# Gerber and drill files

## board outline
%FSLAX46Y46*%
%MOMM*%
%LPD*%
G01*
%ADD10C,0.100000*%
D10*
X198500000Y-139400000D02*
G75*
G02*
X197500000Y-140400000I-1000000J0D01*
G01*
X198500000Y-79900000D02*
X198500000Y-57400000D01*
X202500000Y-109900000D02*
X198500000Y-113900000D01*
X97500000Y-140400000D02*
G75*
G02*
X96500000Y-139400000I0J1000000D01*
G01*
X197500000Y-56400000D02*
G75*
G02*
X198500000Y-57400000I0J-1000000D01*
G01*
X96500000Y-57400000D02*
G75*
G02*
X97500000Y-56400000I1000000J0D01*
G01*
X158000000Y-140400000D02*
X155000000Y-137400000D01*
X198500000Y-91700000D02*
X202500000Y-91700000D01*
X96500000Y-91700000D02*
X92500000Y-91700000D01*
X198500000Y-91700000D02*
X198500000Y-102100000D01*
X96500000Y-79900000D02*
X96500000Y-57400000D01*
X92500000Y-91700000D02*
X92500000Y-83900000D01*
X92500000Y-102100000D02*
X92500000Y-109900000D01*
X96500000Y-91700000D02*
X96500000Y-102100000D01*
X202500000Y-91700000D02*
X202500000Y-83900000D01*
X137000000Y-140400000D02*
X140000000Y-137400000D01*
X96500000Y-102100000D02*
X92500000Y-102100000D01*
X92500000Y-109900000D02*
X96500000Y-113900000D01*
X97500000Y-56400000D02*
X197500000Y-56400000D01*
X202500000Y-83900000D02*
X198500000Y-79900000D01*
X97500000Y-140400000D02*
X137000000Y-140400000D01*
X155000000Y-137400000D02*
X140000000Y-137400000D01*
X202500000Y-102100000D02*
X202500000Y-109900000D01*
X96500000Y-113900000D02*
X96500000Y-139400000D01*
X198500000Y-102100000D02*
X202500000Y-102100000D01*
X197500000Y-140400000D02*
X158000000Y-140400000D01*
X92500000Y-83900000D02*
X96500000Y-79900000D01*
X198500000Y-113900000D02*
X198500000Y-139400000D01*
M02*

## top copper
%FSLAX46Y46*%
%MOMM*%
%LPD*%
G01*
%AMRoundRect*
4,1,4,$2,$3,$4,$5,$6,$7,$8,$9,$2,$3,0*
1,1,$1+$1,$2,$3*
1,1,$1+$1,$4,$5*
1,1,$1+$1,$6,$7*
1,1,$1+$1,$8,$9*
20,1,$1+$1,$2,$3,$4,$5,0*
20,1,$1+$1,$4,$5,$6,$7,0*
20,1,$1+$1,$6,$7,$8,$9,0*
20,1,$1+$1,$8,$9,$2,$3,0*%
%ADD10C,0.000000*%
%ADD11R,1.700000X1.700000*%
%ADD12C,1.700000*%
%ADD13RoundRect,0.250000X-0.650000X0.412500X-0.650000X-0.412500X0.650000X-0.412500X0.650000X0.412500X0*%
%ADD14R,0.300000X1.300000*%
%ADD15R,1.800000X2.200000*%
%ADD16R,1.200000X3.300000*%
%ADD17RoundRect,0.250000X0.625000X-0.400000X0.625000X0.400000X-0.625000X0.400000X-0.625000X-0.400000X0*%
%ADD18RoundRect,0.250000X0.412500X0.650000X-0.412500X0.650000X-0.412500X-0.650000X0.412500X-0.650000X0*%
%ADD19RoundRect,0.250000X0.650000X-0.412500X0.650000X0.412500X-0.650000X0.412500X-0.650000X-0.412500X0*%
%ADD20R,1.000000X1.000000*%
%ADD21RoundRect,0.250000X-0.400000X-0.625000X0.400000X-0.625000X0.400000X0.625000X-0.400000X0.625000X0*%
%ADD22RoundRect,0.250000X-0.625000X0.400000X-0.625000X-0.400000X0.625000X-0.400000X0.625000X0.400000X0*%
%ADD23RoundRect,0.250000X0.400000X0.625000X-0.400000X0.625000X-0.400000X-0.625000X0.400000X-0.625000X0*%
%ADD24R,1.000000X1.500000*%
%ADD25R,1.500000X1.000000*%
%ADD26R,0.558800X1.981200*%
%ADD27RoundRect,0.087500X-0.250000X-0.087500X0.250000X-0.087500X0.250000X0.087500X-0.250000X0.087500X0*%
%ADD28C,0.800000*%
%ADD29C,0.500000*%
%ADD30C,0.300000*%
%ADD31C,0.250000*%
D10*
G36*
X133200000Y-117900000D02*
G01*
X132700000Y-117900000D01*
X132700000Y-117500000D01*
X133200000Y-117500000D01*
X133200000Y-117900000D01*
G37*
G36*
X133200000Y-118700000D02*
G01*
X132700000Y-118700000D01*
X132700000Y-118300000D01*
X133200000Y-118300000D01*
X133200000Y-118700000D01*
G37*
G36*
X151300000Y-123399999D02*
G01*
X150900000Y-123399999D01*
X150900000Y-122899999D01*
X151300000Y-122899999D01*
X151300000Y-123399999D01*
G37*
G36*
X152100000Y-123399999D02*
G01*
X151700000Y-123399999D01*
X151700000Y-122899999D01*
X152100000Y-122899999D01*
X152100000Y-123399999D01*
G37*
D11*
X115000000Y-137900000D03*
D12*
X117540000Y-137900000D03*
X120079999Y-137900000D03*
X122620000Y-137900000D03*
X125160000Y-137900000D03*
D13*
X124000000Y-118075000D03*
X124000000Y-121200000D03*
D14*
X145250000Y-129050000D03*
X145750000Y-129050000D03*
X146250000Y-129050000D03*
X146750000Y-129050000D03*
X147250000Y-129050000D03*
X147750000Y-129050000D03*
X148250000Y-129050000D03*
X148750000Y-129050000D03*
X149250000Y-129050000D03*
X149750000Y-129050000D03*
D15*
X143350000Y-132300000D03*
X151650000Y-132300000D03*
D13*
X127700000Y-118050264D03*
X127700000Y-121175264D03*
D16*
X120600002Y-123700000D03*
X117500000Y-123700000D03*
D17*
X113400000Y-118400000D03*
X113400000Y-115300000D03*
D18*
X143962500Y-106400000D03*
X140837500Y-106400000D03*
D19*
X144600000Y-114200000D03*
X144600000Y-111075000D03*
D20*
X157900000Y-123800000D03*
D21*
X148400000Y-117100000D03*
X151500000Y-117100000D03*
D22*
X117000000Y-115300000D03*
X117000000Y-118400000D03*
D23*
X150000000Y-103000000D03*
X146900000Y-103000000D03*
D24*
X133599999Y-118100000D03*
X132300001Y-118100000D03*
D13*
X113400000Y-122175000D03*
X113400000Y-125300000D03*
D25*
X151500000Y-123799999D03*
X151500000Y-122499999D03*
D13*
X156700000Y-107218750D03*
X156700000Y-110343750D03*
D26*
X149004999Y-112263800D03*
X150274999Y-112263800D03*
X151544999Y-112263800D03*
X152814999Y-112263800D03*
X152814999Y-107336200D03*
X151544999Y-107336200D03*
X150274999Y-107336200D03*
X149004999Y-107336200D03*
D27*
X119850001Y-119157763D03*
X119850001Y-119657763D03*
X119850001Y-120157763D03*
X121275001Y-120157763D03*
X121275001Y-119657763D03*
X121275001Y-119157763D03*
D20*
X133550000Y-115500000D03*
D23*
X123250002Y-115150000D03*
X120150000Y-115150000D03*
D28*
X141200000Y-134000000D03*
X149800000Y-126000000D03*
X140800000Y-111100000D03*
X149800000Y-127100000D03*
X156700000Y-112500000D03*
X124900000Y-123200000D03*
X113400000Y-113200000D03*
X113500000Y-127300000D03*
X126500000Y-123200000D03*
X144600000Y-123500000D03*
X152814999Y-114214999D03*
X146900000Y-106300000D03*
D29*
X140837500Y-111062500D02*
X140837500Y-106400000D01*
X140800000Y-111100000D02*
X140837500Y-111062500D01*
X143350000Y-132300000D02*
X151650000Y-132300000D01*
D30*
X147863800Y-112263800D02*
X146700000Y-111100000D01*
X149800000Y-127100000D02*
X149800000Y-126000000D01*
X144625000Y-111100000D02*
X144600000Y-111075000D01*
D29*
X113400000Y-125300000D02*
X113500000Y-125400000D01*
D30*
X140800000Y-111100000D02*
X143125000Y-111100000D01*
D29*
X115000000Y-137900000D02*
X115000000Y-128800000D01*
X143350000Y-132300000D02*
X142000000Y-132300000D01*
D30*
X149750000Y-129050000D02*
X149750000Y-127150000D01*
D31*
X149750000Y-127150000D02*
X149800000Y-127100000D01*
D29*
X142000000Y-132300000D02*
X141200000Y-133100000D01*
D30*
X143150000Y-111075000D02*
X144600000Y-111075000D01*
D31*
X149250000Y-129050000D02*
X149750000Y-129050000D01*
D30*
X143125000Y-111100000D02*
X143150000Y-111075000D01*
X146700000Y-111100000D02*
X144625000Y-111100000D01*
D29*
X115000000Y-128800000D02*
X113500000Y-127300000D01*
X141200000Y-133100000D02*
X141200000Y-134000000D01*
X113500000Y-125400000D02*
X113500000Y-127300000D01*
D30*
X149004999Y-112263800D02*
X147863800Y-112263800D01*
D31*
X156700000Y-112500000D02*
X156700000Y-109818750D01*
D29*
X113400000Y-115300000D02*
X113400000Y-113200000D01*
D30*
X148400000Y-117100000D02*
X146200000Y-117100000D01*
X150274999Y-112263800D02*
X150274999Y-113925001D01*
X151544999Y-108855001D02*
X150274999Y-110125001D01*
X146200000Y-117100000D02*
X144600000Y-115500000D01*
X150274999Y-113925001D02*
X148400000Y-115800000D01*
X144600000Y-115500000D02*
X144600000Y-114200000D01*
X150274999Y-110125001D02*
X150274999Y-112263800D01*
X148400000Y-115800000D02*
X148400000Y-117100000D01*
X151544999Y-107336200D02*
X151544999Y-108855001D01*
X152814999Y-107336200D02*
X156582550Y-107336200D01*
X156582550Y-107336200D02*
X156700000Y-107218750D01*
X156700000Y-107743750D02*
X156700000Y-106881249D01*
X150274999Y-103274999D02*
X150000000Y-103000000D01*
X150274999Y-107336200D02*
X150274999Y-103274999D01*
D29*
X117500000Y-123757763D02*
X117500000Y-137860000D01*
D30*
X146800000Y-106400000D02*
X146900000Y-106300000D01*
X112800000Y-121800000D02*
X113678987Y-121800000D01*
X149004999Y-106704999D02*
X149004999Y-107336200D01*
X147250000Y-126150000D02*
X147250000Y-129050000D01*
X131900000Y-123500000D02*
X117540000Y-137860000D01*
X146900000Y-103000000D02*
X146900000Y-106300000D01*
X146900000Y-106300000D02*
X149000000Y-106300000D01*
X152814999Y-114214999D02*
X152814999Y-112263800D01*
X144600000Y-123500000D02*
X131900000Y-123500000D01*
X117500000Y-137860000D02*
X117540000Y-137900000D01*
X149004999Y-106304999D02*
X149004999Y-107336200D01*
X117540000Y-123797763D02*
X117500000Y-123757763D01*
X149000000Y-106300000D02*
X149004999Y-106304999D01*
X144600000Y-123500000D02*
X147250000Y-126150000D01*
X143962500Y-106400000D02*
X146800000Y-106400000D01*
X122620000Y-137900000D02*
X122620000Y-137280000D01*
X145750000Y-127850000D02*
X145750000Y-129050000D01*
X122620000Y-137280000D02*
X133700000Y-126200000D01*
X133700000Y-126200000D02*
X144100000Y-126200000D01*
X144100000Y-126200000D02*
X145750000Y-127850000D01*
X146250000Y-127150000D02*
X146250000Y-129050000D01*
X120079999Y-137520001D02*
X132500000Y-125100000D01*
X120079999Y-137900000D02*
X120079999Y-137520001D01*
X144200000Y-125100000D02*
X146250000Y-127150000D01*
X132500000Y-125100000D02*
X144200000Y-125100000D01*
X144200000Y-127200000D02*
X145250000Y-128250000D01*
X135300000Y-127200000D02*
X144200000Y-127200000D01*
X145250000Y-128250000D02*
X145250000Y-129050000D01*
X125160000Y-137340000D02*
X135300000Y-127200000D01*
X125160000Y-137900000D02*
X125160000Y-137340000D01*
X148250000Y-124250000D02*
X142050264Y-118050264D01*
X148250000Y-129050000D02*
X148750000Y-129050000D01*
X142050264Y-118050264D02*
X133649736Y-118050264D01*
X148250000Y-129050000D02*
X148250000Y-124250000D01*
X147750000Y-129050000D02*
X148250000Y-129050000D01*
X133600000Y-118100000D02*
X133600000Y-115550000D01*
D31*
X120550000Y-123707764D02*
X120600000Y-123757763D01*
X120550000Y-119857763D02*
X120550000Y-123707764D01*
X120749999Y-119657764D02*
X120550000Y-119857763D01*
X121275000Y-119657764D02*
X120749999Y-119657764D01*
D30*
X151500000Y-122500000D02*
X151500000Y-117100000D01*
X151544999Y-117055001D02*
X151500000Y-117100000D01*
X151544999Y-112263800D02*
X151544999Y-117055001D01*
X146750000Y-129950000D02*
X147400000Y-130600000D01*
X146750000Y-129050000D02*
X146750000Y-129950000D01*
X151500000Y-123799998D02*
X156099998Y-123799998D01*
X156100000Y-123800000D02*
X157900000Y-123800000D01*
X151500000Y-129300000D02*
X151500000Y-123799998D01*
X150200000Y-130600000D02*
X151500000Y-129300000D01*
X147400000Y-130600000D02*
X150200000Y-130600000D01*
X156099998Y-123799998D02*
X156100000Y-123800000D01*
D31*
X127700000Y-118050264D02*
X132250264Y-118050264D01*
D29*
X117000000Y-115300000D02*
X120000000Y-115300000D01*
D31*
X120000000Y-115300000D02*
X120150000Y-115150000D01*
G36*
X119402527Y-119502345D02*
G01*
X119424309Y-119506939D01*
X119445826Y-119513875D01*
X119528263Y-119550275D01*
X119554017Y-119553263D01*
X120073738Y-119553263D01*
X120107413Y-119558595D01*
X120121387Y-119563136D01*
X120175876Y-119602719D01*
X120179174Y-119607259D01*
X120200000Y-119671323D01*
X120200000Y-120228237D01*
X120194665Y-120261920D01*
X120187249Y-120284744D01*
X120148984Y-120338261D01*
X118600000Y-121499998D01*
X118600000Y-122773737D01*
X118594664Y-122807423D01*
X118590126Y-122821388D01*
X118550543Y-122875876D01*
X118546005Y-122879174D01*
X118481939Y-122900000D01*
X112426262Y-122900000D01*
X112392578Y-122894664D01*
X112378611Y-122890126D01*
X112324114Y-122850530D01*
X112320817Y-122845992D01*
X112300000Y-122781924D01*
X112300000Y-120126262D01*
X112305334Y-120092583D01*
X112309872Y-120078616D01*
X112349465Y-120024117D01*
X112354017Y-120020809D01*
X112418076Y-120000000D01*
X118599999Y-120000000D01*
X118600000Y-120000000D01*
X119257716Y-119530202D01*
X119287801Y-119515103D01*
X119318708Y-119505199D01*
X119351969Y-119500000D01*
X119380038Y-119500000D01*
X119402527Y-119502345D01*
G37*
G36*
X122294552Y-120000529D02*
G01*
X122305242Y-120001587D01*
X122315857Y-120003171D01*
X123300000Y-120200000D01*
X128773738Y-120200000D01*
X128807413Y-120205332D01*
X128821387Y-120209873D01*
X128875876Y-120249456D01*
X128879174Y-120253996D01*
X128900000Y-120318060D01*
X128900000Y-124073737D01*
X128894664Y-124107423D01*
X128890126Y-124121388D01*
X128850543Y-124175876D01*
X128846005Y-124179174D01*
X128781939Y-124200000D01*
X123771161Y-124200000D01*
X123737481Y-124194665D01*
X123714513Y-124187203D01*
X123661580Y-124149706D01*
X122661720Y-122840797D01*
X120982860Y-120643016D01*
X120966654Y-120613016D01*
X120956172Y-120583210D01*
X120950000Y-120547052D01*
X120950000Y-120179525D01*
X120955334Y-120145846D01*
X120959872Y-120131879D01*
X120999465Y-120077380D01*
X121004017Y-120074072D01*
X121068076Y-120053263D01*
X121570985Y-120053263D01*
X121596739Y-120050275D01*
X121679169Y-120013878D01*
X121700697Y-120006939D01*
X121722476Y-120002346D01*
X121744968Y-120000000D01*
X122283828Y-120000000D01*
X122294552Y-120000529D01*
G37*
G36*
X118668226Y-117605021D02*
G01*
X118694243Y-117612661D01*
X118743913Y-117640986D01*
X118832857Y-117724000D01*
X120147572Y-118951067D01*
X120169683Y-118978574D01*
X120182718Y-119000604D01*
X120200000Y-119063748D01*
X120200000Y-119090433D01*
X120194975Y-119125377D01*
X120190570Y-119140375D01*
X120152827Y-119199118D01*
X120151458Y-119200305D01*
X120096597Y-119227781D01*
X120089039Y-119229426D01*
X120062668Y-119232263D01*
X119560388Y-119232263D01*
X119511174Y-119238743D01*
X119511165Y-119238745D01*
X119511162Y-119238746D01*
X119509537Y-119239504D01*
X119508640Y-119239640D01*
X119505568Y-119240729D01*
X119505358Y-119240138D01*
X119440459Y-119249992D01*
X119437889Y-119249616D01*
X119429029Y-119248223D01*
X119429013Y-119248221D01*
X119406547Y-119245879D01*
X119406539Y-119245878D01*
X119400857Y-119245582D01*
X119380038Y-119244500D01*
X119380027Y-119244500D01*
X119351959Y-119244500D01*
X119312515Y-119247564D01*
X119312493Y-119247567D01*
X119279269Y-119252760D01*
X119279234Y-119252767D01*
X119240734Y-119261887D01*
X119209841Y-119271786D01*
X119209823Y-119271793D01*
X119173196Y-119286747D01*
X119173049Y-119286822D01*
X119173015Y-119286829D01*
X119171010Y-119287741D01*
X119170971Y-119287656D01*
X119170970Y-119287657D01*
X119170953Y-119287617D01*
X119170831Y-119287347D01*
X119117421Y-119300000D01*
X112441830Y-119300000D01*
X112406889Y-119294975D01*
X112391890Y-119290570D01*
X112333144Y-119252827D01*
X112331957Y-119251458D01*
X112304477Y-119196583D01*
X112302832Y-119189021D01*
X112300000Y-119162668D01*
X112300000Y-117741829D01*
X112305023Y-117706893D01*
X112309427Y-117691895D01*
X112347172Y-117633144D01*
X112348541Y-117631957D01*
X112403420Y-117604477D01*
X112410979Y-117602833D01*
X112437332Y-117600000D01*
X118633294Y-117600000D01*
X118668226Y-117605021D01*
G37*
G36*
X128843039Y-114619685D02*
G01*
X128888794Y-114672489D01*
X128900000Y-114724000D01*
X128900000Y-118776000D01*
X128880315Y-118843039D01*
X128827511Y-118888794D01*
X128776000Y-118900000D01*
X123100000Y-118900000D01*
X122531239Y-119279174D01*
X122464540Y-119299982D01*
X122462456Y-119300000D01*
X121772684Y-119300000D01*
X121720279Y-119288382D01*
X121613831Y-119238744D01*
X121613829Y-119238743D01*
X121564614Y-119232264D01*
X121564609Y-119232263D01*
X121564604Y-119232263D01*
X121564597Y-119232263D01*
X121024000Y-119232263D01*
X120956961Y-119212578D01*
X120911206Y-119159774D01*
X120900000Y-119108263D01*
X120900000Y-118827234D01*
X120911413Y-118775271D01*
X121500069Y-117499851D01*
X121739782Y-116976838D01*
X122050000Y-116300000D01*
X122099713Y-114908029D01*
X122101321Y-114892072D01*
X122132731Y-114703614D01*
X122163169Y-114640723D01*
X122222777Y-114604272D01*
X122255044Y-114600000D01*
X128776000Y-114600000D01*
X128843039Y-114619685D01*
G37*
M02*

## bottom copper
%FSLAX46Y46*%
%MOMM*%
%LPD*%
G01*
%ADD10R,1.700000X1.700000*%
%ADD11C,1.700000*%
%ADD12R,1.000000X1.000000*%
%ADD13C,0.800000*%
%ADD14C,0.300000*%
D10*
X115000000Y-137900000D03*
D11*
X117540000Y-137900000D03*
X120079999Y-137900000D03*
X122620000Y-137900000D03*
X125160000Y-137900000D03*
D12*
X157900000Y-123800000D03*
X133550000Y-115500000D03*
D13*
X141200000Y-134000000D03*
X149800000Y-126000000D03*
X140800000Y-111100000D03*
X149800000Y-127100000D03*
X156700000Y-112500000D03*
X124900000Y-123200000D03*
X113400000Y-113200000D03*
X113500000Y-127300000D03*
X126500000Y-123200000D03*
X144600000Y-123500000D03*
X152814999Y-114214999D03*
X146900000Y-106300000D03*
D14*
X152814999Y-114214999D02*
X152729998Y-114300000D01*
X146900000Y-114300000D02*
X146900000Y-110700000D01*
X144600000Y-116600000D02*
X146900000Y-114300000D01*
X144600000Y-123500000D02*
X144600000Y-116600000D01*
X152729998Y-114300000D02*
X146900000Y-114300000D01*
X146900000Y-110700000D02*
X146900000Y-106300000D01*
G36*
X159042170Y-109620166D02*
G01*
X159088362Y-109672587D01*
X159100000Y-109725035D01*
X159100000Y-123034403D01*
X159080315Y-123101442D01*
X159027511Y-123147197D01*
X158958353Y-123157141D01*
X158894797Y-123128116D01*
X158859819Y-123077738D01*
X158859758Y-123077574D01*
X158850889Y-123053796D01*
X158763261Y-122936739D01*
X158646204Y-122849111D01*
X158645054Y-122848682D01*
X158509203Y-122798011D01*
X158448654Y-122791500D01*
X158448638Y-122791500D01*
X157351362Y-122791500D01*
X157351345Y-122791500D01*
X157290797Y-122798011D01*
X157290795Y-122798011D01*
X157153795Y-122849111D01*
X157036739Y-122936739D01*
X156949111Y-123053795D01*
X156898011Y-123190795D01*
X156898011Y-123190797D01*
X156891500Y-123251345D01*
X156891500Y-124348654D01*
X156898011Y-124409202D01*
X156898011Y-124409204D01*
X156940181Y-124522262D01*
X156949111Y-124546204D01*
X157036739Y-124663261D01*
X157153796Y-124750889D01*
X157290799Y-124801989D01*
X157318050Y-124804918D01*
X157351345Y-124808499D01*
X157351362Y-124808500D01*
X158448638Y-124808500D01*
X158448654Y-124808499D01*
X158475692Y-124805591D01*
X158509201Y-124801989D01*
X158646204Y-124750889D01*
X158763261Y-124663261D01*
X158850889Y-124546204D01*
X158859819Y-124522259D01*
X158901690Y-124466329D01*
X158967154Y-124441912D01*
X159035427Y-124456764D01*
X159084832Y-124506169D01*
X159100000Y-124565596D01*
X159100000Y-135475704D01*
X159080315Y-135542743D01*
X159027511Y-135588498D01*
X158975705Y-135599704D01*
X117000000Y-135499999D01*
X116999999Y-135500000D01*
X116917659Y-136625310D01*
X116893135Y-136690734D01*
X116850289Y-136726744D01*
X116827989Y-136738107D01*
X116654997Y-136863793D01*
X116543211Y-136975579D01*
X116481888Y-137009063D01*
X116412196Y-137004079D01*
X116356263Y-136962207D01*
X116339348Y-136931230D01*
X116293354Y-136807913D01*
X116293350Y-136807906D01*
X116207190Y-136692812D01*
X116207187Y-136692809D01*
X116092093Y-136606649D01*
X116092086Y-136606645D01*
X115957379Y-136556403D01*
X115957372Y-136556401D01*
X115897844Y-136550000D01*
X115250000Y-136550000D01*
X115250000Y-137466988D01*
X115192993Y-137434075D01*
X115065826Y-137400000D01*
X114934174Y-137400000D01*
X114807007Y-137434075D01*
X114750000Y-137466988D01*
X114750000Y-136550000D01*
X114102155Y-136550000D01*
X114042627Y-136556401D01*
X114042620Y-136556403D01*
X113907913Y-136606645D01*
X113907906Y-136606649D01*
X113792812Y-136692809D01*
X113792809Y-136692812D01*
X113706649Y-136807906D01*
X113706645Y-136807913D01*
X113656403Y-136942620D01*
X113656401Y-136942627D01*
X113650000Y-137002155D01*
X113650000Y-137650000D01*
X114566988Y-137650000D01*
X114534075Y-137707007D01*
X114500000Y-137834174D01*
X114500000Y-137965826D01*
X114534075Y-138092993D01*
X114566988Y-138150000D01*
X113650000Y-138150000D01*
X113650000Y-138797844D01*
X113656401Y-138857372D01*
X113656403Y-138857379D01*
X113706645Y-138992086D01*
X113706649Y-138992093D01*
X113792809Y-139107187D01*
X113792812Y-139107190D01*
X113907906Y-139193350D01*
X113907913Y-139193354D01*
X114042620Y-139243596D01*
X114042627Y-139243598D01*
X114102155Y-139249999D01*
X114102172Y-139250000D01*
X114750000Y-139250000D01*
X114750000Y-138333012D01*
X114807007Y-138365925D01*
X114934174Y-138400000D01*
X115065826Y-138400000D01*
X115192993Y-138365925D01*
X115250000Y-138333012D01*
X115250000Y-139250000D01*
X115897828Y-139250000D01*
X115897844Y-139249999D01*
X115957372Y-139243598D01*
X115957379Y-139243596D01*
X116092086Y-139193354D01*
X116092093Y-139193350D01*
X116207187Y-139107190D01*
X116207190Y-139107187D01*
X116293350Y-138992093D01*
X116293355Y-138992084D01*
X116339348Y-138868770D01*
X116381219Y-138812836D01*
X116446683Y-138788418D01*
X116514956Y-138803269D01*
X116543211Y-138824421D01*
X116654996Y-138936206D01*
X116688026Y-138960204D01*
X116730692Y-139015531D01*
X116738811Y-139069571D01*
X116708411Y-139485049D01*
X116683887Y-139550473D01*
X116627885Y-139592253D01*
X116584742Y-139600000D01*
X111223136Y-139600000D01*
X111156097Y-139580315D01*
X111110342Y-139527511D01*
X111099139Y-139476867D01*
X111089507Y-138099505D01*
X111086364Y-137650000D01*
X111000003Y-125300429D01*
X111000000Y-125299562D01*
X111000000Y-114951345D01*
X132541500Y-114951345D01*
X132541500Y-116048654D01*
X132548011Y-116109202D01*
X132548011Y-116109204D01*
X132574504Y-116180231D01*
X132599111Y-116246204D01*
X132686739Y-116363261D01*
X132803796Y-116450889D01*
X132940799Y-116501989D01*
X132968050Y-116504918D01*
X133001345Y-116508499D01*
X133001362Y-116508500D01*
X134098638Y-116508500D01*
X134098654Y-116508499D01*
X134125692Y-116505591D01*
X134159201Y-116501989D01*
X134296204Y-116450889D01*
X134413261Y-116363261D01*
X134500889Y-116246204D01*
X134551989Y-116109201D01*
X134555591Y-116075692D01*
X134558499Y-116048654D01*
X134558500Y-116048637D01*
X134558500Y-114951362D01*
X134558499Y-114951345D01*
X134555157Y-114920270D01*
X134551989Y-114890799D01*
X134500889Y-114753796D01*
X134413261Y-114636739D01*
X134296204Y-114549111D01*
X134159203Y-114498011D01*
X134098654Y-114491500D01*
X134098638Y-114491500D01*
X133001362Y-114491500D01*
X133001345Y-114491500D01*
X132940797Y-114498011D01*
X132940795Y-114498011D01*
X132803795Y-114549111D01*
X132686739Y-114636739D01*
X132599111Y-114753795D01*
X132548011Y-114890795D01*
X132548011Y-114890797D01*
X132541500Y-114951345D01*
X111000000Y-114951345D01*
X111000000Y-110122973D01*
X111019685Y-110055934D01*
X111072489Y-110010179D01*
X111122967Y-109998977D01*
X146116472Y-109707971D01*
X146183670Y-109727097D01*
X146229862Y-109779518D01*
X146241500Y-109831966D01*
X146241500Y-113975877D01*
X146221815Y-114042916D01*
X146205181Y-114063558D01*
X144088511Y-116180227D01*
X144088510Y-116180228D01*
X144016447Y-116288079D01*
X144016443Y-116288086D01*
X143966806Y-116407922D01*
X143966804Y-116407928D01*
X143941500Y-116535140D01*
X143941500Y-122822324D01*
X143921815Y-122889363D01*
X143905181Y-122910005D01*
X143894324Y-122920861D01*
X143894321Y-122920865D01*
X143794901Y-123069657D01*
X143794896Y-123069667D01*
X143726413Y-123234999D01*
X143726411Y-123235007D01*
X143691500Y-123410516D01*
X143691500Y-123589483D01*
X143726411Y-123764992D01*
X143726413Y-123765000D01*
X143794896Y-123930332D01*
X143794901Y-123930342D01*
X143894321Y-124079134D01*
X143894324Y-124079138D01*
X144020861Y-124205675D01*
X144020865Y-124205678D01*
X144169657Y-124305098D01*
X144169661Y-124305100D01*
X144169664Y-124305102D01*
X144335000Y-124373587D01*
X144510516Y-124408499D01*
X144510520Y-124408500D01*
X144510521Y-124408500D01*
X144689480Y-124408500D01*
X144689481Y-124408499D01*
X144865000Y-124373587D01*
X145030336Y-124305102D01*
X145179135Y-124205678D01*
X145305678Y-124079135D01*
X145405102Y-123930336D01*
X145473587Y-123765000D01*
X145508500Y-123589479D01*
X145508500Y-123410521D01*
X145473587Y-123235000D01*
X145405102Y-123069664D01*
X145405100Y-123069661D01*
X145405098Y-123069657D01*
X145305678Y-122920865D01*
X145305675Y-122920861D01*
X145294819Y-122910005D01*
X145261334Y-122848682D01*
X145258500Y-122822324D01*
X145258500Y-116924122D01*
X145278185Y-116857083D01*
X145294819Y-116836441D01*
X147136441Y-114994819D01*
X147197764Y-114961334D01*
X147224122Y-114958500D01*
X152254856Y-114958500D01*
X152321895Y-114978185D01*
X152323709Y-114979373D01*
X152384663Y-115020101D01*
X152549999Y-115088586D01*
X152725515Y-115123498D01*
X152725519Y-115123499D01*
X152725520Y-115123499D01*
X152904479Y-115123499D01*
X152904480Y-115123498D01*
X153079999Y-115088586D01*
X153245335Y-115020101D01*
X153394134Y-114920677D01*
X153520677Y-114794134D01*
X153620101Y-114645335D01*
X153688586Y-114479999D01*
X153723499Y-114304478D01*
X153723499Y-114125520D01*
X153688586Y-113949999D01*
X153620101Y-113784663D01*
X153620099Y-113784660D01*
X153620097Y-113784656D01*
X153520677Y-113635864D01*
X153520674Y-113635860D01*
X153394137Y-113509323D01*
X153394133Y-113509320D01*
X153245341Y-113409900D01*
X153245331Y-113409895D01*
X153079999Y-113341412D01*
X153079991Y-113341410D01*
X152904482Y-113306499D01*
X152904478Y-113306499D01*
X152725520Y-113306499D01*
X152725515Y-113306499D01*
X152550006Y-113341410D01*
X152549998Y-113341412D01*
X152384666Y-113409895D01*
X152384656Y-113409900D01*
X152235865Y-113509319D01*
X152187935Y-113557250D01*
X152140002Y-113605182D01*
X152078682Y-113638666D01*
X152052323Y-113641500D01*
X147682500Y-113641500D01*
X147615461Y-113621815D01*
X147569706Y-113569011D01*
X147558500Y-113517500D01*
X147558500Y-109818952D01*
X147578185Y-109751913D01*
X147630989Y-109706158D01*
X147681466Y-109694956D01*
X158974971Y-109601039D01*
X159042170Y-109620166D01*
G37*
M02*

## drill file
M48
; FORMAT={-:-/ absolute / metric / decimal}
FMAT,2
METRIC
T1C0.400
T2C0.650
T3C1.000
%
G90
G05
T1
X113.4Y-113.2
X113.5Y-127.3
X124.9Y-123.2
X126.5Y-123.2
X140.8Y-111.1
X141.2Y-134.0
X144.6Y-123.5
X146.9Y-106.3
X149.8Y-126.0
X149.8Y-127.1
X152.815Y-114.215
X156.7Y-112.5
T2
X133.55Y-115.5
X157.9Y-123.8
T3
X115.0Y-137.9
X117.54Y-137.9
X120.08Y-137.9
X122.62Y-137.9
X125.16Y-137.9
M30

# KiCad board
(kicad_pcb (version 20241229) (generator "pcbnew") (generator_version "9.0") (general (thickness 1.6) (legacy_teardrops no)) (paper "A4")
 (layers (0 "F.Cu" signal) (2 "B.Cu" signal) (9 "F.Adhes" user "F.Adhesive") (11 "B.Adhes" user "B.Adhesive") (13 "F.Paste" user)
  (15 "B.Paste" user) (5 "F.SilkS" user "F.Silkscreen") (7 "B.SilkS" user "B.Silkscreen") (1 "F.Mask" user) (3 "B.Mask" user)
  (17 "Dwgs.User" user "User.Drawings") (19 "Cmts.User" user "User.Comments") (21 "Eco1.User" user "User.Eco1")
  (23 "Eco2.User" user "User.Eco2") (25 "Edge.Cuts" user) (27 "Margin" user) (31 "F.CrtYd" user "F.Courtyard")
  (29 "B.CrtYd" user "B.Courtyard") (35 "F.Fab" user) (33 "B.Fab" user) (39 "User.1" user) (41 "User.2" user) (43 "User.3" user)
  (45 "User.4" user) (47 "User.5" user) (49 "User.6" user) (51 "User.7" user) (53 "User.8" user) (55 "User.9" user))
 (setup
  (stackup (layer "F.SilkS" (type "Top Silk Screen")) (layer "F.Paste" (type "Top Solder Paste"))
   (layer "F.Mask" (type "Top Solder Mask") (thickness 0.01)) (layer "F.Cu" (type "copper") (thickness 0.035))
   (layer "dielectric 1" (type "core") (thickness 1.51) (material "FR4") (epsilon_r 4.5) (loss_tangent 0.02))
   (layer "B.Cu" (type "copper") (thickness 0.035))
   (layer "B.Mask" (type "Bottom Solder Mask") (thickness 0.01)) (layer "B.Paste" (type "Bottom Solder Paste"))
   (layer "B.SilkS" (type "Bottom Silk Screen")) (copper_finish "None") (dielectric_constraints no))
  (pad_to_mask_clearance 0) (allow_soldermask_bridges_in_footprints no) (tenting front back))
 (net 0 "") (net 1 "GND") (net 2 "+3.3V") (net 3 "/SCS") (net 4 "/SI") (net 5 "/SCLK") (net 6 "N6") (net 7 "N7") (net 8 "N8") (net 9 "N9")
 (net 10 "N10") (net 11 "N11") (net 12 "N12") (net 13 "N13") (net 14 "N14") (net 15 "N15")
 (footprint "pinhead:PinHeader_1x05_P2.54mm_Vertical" (layer "F.Cu") (at 115 137.9 90)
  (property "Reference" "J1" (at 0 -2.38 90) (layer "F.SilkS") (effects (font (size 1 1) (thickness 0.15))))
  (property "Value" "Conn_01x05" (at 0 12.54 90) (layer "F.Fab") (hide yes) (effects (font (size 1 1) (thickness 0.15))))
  (pad "1" thru_hole rect (at 0 0 90) (size 1.7 1.7) (drill 1) (layers "*.Cu" "*.Mask") (remove_unused_layers no) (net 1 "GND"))
  (pad "2" thru_hole circle (at 0 2.54 90) (size 1.7 1.7) (drill 1) (layers "*.Cu" "*.Mask") (remove_unused_layers no) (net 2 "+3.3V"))
  (pad "3" thru_hole circle (at 0 5.079999 90) (size 1.7 1.7) (drill 1) (layers "*.Cu" "*.Mask") (remove_unused_layers no) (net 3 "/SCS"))
  (pad "4" thru_hole circle (at 0 7.62 90) (size 1.7 1.7) (drill 1) (layers "*.Cu" "*.Mask") (remove_unused_layers no) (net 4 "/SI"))
  (pad "5" thru_hole circle (at 0 10.16 90) (size 1.7 1.7) (drill 1) (layers "*.Cu" "*.Mask") (remove_unused_layers no) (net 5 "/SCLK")))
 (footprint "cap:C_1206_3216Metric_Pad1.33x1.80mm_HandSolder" (layer "F.Cu") (at 124 119.6375 -90)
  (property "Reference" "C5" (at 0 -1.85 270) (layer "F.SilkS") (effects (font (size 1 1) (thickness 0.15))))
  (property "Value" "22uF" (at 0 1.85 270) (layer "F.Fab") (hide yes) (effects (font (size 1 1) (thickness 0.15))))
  (pad "1" smd roundrect (at -1.5625 0 270) (size 1.325 1.8) (layers "F.Cu" "F.Mask" "F.Paste") (roundrect_rratio 0.188679) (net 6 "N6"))
  (pad "2" smd roundrect (at 1.5625 0 270) (size 1.325 1.8) (layers "F.Cu" "F.Mask" "F.Paste") (roundrect_rratio 0.188679) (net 1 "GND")))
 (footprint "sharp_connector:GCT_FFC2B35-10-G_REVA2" (layer "F.Cu") (at 147.5 132.3)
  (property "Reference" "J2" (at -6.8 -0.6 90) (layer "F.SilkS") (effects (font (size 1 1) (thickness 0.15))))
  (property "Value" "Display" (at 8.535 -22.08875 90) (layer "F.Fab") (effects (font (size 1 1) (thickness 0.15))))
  (pad "1" smd rect (at -2.25 -3.25) (size 0.3 1.3) (layers "F.Cu" "F.Mask" "F.Paste") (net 5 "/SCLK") (solder_mask_margin 0))
  (pad "2" smd rect (at -1.75 -3.25) (size 0.3 1.3) (layers "F.Cu" "F.Mask" "F.Paste") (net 4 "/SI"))
  (pad "3" smd rect (at -1.25 -3.25) (size 0.3 1.3) (layers "F.Cu" "F.Mask" "F.Paste") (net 3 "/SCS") (solder_mask_margin 0))
  (pad "4" smd rect (at -0.75 -3.25) (size 0.3 1.3) (layers "F.Cu" "F.Mask" "F.Paste") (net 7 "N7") (solder_mask_margin 0))
  (pad "5" smd rect (at -0.25 -3.25) (size 0.3 1.3) (layers "F.Cu" "F.Mask" "F.Paste") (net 2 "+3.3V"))
  (pad "6" smd rect (at 0.25 -3.25) (size 0.3 1.3) (layers "F.Cu" "F.Mask" "F.Paste") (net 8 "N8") (solder_mask_margin 0))
  (pad "7" smd rect (at 0.75 -3.25) (size 0.3 1.3) (layers "F.Cu" "F.Mask" "F.Paste") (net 8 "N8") (solder_mask_margin 0))
  (pad "8" smd rect (at 1.25 -3.25) (size 0.3 1.3) (layers "F.Cu" "F.Mask" "F.Paste") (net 8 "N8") (solder_mask_margin 0))
  (pad "9" smd rect (at 1.75 -3.25) (size 0.3 1.3) (layers "F.Cu" "F.Mask" "F.Paste") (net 1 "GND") (solder_mask_margin 0))
  (pad "10" smd rect (at 2.25 -3.25) (size 0.3 1.3) (layers "F.Cu" "F.Mask" "F.Paste") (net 1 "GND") (solder_mask_margin 0))
  (pad "MP1" smd rect (at -4.15 0) (size 1.8 2.2) (layers "F.Cu" "F.Mask" "F.Paste") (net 1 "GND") (solder_mask_margin 0))
  (pad "MP2" smd rect (at 4.15 0) (size 1.8 2.2) (layers "F.Cu" "F.Mask" "F.Paste") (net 1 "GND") (solder_mask_margin 0)))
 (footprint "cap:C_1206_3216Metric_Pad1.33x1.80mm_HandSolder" (layer "F.Cu") (at 127.7 119.612764 -90)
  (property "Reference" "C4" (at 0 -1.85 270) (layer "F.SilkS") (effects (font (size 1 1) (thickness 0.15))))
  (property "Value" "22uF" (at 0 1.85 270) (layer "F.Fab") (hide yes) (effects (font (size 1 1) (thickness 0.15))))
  (pad "1" smd roundrect (at -1.5625 0 270) (size 1.325 1.8) (layers "F.Cu" "F.Mask" "F.Paste") (roundrect_rratio 0.188679) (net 6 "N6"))
  (pad "2" smd roundrect (at 1.5625 0 270) (size 1.325 1.8) (layers "F.Cu" "F.Mask" "F.Paste") (roundrect_rratio 0.188679) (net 1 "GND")))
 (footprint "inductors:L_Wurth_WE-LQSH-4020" (layer "F.Cu") (at 119.050001 123.7 180)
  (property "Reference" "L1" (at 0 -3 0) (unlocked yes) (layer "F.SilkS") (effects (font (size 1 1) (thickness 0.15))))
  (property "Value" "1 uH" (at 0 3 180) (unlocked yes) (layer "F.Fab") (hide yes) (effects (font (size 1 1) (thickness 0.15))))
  (pad "1" smd rect (at -1.550001 0 180) (size 1.2 3.3) (layers "F.Cu" "F.Mask" "F.Paste") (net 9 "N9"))
  (pad "2" smd rect (at 1.550001 0 180) (size 1.2 3.3) (layers "F.Cu" "F.Mask" "F.Paste") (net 2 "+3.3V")))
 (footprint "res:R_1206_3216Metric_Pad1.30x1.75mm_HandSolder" (layer "F.Cu") (at 113.4 116.85 90)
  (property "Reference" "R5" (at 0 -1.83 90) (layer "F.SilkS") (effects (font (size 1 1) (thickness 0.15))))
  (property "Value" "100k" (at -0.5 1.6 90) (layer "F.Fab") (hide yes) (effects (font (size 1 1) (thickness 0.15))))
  (pad "1" smd roundrect (at -1.55 0 90) (size 1.3 1.75) (layers "F.Cu" "F.Mask" "F.Paste") (roundrect_rratio 0.192308) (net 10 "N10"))
  (pad "2" smd roundrect (at 1.55 0 90) (size 1.3 1.75) (layers "F.Cu" "F.Mask" "F.Paste") (roundrect_rratio 0.192308) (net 1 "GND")))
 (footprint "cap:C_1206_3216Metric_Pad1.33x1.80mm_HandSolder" (layer "F.Cu") (at 142.4 106.4 180)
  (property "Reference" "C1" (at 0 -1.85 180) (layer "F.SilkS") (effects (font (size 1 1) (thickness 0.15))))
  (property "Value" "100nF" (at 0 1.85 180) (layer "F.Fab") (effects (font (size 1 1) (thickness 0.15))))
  (pad "1" smd roundrect (at -1.5625 0 180) (size 1.325 1.8) (layers "F.Cu" "F.Mask" "F.Paste") (roundrect_rratio 0.188679) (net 2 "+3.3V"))
  (pad "2" smd roundrect (at 1.5625 0 180) (size 1.325 1.8) (layers "F.Cu" "F.Mask" "F.Paste") (roundrect_rratio 0.188679) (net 1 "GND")))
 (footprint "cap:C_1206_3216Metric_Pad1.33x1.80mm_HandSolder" (layer "F.Cu") (at 144.6 112.6375 90)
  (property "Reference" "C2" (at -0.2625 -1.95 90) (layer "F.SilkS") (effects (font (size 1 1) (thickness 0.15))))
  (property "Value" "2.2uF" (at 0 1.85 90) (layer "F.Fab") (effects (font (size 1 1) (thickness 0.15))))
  (pad "1" smd roundrect (at -1.5625 0 90) (size 1.325 1.8) (layers "F.Cu" "F.Mask" "F.Paste") (roundrect_rratio 0.188679) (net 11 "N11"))
  (pad "2" smd roundrect (at 1.5625 0 90) (size 1.325 1.8) (layers "F.Cu" "F.Mask" "F.Paste") (roundrect_rratio 0.188679) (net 1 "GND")))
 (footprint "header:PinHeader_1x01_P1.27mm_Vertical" (layer "F.Cu") (at 157.9 123.8)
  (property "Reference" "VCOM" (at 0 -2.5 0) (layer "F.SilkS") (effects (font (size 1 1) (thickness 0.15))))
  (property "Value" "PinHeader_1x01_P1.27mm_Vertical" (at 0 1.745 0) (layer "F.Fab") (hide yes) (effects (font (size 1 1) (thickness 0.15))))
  (pad "1" thru_hole rect (at 0 0) (size 1 1) (drill 0.65) (layers "*.Cu" "*.Mask") (remove_unused_layers no) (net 7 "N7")))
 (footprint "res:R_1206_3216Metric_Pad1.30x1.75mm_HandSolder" (layer "F.Cu") (at 149.95 117.1)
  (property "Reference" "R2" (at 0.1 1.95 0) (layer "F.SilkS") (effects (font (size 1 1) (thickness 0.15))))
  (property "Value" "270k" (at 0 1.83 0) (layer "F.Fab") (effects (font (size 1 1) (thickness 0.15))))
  (pad "1" smd roundrect (at -1.55 0) (size 1.3 1.75) (layers "F.Cu" "F.Mask" "F.Paste") (roundrect_rratio 0.192308) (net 11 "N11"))
  (pad "2" smd roundrect (at 1.55 0) (size 1.3 1.75) (layers "F.Cu" "F.Mask" "F.Paste") (roundrect_rratio 0.192308) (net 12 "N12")))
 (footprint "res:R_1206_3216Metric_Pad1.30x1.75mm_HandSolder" (layer "F.Cu") (at 117 116.85 -90)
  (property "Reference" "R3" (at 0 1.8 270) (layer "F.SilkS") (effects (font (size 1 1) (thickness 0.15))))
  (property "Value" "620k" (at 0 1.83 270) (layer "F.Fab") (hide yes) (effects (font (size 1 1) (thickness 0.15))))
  (pad "1" smd roundrect (at -1.55 0 270) (size 1.3 1.75) (layers "F.Cu" "F.Mask" "F.Paste") (roundrect_rratio 0.192308) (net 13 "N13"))
  (pad "2" smd roundrect (at 1.55 0 270) (size 1.3 1.75) (layers "F.Cu" "F.Mask" "F.Paste") (roundrect_rratio 0.192308) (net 10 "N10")))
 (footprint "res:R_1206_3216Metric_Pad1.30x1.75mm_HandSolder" (layer "F.Cu") (at 148.45 103 180)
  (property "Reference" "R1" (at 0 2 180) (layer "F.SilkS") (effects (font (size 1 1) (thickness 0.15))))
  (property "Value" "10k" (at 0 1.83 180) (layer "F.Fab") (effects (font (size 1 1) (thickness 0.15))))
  (pad "1" smd roundrect (at -1.55 0 180) (size 1.3 1.75) (layers "F.Cu" "F.Mask" "F.Paste") (roundrect_rratio 0.192308) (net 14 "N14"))
  (pad "2" smd roundrect (at 1.55 0 180) (size 1.3 1.75) (layers "F.Cu" "F.Mask" "F.Paste") (roundrect_rratio 0.192308) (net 2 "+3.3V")))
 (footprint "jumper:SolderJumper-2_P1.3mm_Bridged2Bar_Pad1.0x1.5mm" (layer "F.Cu") (at 132.95 118.1 180)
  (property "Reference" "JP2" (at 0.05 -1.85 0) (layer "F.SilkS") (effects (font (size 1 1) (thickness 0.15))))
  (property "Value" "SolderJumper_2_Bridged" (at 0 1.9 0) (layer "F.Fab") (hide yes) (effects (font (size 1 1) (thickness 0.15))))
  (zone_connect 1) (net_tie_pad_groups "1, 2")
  (fp_poly (pts (xy -0.25 0.2) (xy 0.25 0.2) (xy 0.25 0.6) (xy -0.25 0.6)) (stroke (width 0) (type solid)) (fill yes) (layer "F.Cu"))
  (fp_poly (pts (xy -0.25 -0.6) (xy 0.25 -0.6) (xy 0.25 -0.2) (xy -0.25 -0.2)) (stroke (width 0) (type solid)) (fill yes) (layer "F.Cu"))
  (pad "1" smd rect (at -0.649999 0 180) (size 1 1.5) (layers "F.Cu" "F.Mask") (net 8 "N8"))
  (pad "2" smd rect (at 0.649999 0 180) (size 1 1.5) (layers "F.Cu" "F.Mask") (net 6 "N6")))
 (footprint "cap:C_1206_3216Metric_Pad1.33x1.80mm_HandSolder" (layer "F.Cu") (at 113.4 123.7375 -90)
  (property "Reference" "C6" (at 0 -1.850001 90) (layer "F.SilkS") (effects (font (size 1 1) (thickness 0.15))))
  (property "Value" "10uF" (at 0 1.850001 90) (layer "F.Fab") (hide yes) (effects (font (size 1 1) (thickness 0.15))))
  (pad "1" smd roundrect (at -1.5625 0 270) (size 1.325 1.8) (layers "F.Cu" "F.Mask" "F.Paste") (roundrect_rratio 0.188679) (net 2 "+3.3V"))
  (pad "2" smd roundrect (at 1.5625 0 270) (size 1.325 1.8) (layers "F.Cu" "F.Mask" "F.Paste") (roundrect_rratio 0.188679) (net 1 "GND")))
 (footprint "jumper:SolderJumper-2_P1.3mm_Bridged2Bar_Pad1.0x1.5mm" (layer "F.Cu") (at 151.5 123.149999 90)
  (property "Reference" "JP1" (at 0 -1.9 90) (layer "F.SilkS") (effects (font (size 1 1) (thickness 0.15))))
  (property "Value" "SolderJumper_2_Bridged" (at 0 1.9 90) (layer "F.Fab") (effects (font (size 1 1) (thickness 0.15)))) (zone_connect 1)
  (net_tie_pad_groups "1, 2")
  (fp_poly (pts (xy -0.25 -0.6) (xy 0.25 -0.6) (xy 0.25 -0.2) (xy -0.25 -0.2)) (stroke (width 0) (type solid)) (fill yes) (layer "F.Cu"))
  (fp_poly (pts (xy -0.25 0.2) (xy 0.25 0.2) (xy 0.25 0.6) (xy -0.25 0.6)) (stroke (width 0) (type solid)) (fill yes) (layer "F.Cu"))
  (pad "1" smd rect (at -0.65 0 90) (size 1 1.5) (layers "F.Cu" "F.Mask") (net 7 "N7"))
  (pad "2" smd rect (at 0.65 0 90) (size 1 1.5) (layers "F.Cu" "F.Mask") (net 12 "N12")))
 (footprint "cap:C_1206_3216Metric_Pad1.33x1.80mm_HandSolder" (layer "F.Cu") (at 156.7 108.78125 -90)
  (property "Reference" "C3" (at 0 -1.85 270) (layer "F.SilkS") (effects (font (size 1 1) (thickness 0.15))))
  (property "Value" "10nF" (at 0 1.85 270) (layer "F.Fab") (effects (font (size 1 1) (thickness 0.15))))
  (pad "1" smd roundrect (at -1.5625 0 270) (size 1.325 1.8) (layers "F.Cu" "F.Mask" "F.Paste") (roundrect_rratio 0.188679) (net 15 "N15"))
  (pad "2" smd roundrect (at 1.5625 0 270) (size 1.325 1.8) (layers "F.Cu" "F.Mask" "F.Paste") (roundrect_rratio 0.188679) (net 1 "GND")))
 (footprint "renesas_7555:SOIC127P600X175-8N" (layer "F.Cu") (at 150.909999 109.8 90)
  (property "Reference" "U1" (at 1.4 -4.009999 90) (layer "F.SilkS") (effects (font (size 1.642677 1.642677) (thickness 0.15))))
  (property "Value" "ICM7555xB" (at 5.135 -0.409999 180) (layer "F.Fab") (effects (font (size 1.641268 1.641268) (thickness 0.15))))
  (pad "1" smd rect (at -2.4638 -1.905 90) (size 1.9812 0.5588) (layers "F.Cu" "F.Mask" "F.Paste") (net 1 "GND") (solder_mask_margin 0.102))
  (pad "2" smd rect (at -2.4638 -0.635 90) (size 1.9812 0.5588) (layers "F.Cu" "F.Mask" "F.Paste") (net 11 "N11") (solder_mask_margin 0.102))
  (pad "3" smd rect (at -2.4638 0.635 90) (size 1.9812 0.5588) (layers "F.Cu" "F.Mask" "F.Paste") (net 12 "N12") (solder_mask_margin 0.102))
  (pad "4" smd rect (at -2.4638 1.905 90) (size 1.9812 0.5588) (layers "F.Cu" "F.Mask" "F.Paste") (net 2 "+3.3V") (solder_mask_margin 0.102))
  (pad "5" smd rect (at 2.4638 1.905 90) (size 1.9812 0.5588) (layers "F.Cu" "F.Mask" "F.Paste") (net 15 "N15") (solder_mask_margin 0.102))
  (pad "6" smd rect (at 2.4638 0.635 90) (size 1.9812 0.5588) (layers "F.Cu" "F.Mask" "F.Paste") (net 11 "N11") (solder_mask_margin 0.102))
  (pad "7" smd rect (at 2.4638 -0.635 90) (size 1.9812 0.5588) (layers "F.Cu" "F.Mask" "F.Paste") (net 14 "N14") (solder_mask_margin 0.102))
  (pad "8" smd rect (at 2.4638 -1.905 90) (size 1.9812 0.5588) (layers "F.Cu" "F.Mask" "F.Paste") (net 2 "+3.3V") (solder_mask_margin 0.102)))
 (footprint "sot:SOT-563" (layer "F.Cu") (at 120.562501 119.657763)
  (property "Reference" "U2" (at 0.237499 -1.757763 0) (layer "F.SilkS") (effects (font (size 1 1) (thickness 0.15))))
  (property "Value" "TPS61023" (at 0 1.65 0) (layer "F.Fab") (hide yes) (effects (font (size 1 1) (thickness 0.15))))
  (pad "1" smd roundrect (at -0.7125 -0.5) (size 0.675 0.35) (layers "F.Cu" "F.Mask" "F.Paste") (roundrect_rratio 0.25) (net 10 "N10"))
  (pad "2" smd roundrect (at -0.7125 0) (size 0.675 0.35) (layers "F.Cu" "F.Mask" "F.Paste") (roundrect_rratio 0.25) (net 2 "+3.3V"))
  (pad "3" smd roundrect (at -0.7125 0.5) (size 0.675 0.35) (layers "F.Cu" "F.Mask" "F.Paste") (roundrect_rratio 0.25) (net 2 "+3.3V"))
  (pad "4" smd roundrect (at 0.7125 0.5) (size 0.675 0.35) (layers "F.Cu" "F.Mask" "F.Paste") (roundrect_rratio 0.25) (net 1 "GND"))
  (pad "5" smd roundrect (at 0.7125 0) (size 0.675 0.35) (layers "F.Cu" "F.Mask" "F.Paste") (roundrect_rratio 0.25) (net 9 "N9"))
  (pad "6" smd roundrect (at 0.7125 -0.5) (size 0.675 0.35) (layers "F.Cu" "F.Mask" "F.Paste") (roundrect_rratio 0.25) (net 6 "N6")))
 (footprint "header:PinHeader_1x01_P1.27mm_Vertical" (layer "F.Cu") (at 133.55 115.5)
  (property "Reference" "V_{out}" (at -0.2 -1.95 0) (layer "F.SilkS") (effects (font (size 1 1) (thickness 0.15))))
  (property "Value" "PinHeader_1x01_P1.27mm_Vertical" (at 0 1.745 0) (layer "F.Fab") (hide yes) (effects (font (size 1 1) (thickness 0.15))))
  (pad "1" thru_hole rect (at 0 0) (size 1 1) (drill 0.65) (layers "*.Cu" "*.Mask") (remove_unused_layers no) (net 8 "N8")))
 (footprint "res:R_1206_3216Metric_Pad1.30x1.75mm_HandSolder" (layer "F.Cu") (at 121.700001 115.15 180)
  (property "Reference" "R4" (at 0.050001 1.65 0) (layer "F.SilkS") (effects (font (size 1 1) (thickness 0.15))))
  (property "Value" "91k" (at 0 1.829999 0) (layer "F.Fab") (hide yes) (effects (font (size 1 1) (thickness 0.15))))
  (pad "1" smd roundrect (at -1.550001 0 180) (size 1.3 1.75) (layers "F.Cu" "F.Mask" "F.Paste") (roundrect_rratio 0.192308) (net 6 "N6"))
  (pad "2" smd roundrect (at 1.550001 0 180) (size 1.3 1.75) (layers "F.Cu" "F.Mask" "F.Paste") (roundrect_rratio 0.192308) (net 13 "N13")))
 (gr_arc (start 198.5 139.4) (mid 198.207107 140.107107) (end 197.5 140.4) (stroke (width 0.1) (type default)) (layer "Edge.Cuts"))
 (gr_line (start 198.5 79.9) (end 198.5 57.4) (stroke (width 0.1) (type default)) (layer "Edge.Cuts"))
 (gr_line (start 202.5 109.9) (end 198.5 113.9) (stroke (width 0.1) (type default)) (layer "Edge.Cuts"))
 (gr_arc (start 97.5 140.4) (mid 96.792893 140.107107) (end 96.5 139.4) (stroke (width 0.1) (type default)) (layer "Edge.Cuts"))
 (gr_arc (start 197.5 56.4) (mid 198.207107 56.692893) (end 198.5 57.4) (stroke (width 0.1) (type default)) (layer "Edge.Cuts"))
 (gr_arc (start 96.5 57.4) (mid 96.792893 56.692893) (end 97.5 56.4) (stroke (width 0.1) (type default)) (layer "Edge.Cuts"))
 (gr_line (start 158 140.4) (end 155 137.4) (stroke (width 0.1) (type default)) (layer "Edge.Cuts"))
 (gr_line (start 198.5 91.7) (end 202.5 91.7) (stroke (width 0.1) (type default)) (layer "Edge.Cuts"))
 (gr_line (start 96.5 91.7) (end 92.5 91.7) (stroke (width 0.1) (type default)) (layer "Edge.Cuts"))
 (gr_line (start 198.5 91.7) (end 198.5 102.1) (stroke (width 0.1) (type default)) (layer "Edge.Cuts"))
 (gr_line (start 96.5 79.9) (end 96.5 57.4) (stroke (width 0.1) (type default)) (layer "Edge.Cuts"))
 (gr_line (start 92.5 91.7) (end 92.5 83.9) (stroke (width 0.1) (type default)) (layer "Edge.Cuts"))
 (gr_line (start 92.5 102.1) (end 92.5 109.9) (stroke (width 0.1) (type default)) (layer "Edge.Cuts"))
 (gr_line (start 96.5 91.7) (end 96.5 102.1) (stroke (width 0.1) (type default)) (layer "Edge.Cuts"))
 (gr_line (start 202.5 91.7) (end 202.5 83.9) (stroke (width 0.1) (type default)) (layer "Edge.Cuts"))
 (gr_line (start 137 140.4) (end 140 137.4) (stroke (width 0.1) (type default)) (layer "Edge.Cuts"))
 (gr_line (start 96.5 102.1) (end 92.5 102.1) (stroke (width 0.1) (type default)) (layer "Edge.Cuts"))
 (gr_line (start 92.5 109.9) (end 96.5 113.9) (stroke (width 0.1) (type default)) (layer "Edge.Cuts"))
 (gr_line (start 97.5 56.4) (end 197.5 56.4) (stroke (width 0.1) (type default)) (layer "Edge.Cuts"))
 (gr_line (start 202.5 83.9) (end 198.5 79.9) (stroke (width 0.1) (type default)) (layer "Edge.Cuts"))
 (gr_line (start 97.5 140.4) (end 137 140.4) (stroke (width 0.1) (type default)) (layer "Edge.Cuts"))
 (gr_line (start 155 137.4) (end 140 137.4) (stroke (width 0.1) (type default)) (layer "Edge.Cuts"))
 (gr_line (start 202.5 102.1) (end 202.5 109.9) (stroke (width 0.1) (type default)) (layer "Edge.Cuts"))
 (gr_line (start 96.5 113.9) (end 96.5 139.4) (stroke (width 0.1) (type default)) (layer "Edge.Cuts"))
 (gr_line (start 198.5 102.1) (end 202.5 102.1) (stroke (width 0.1) (type default)) (layer "Edge.Cuts"))
 (gr_line (start 197.5 140.4) (end 158 140.4) (stroke (width 0.1) (type default)) (layer "Edge.Cuts"))
 (gr_line (start 92.5 83.9) (end 96.5 79.9) (stroke (width 0.1) (type default)) (layer "Edge.Cuts"))
 (gr_line (start 198.5 113.9) (end 198.5 139.4) (stroke (width 0.1) (type default)) (layer "Edge.Cuts"))
 (segment (start 140.8375 111.0625) (end 140.8375 106.4) (width 0.5) (layer "F.Cu") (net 1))
 (segment (start 140.8 111.1) (end 140.8375 111.0625) (width 0.5) (layer "F.Cu") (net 1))
 (segment (start 143.35 132.3) (end 151.65 132.3) (width 0.5) (layer "F.Cu") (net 1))
 (segment (start 147.8638 112.2638) (end 146.7 111.1) (width 0.3) (layer "F.Cu") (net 1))
 (segment (start 149.8 127.1) (end 149.8 126) (width 0.3) (layer "F.Cu") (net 1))
 (segment (start 144.625 111.1) (end 144.6 111.075) (width 0.3) (layer "F.Cu") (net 1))
 (segment (start 113.4 125.3) (end 113.5 125.4) (width 0.5) (layer "F.Cu") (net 1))
 (segment (start 140.8 111.1) (end 143.125 111.1) (width 0.3) (layer "F.Cu") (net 1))
 (segment (start 115 137.9) (end 115 128.8) (width 0.5) (layer "F.Cu") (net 1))
 (segment (start 143.35 132.3) (end 142 132.3) (width 0.5) (layer "F.Cu") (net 1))
 (segment (start 149.75 129.05) (end 149.75 127.15) (width 0.3) (layer "F.Cu") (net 1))
 (segment (start 149.75 127.15) (end 149.8 127.1) (width 0.25) (layer "F.Cu") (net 1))
 (segment (start 142 132.3) (end 141.2 133.1) (width 0.5) (layer "F.Cu") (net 1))
 (segment (start 143.15 111.075) (end 144.6 111.075) (width 0.3) (layer "F.Cu") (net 1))
 (segment (start 149.25 129.05) (end 149.75 129.05) (width 0.25) (layer "F.Cu") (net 1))
 (segment (start 143.125 111.1) (end 143.15 111.075) (width 0.3) (layer "F.Cu") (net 1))
 (segment (start 146.7 111.1) (end 144.625 111.1) (width 0.3) (layer "F.Cu") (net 1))
 (segment (start 115 128.8) (end 113.5 127.3) (width 0.5) (layer "F.Cu") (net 1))
 (segment (start 141.2 133.1) (end 141.2 134) (width 0.5) (layer "F.Cu") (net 1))
 (segment (start 113.5 125.4) (end 113.5 127.3) (width 0.5) (layer "F.Cu") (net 1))
 (segment (start 149.004999 112.2638) (end 147.8638 112.2638) (width 0.3) (layer "F.Cu") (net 1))
 (segment (start 156.7 112.5) (end 156.7 109.81875) (width 0.25) (layer "F.Cu") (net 1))
 (segment (start 113.4 115.3) (end 113.4 113.2) (width 0.5) (layer "F.Cu") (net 1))
 (via (at 141.2 134) (size 0.8) (drill 0.4) (layers "F.Cu" "B.Cu") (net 1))
 (via (at 149.8 126) (size 0.8) (drill 0.4) (layers "F.Cu" "B.Cu") (free yes) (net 1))
 (via (at 140.8 111.1) (size 0.8) (drill 0.4) (layers "F.Cu" "B.Cu") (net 1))
 (via (at 149.8 127.1) (size 0.8) (drill 0.4) (layers "F.Cu" "B.Cu") (free yes) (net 1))
 (via (at 156.7 112.5) (size 0.8) (drill 0.4) (layers "F.Cu" "B.Cu") (free yes) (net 1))
 (via (at 124.9 123.2) (size 0.8) (drill 0.4) (layers "F.Cu" "B.Cu") (free yes) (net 1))
 (via (at 113.4 113.2) (size 0.8) (drill 0.4) (layers "F.Cu" "B.Cu") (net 1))
 (via (at 113.5 127.3) (size 0.8) (drill 0.4) (layers "F.Cu" "B.Cu") (free yes) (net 1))
 (via (at 126.5 123.2) (size 0.8) (drill 0.4) (layers "F.Cu" "B.Cu") (free yes) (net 1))
 (segment (start 148.4 117.1) (end 146.2 117.1) (width 0.3) (layer "F.Cu") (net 11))
 (segment (start 150.274999 112.2638) (end 150.274999 113.925001) (width 0.3) (layer "F.Cu") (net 11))
 (segment (start 151.544999 108.855001) (end 150.274999 110.125001) (width 0.3) (layer "F.Cu") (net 11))
 (segment (start 146.2 117.1) (end 144.6 115.5) (width 0.3) (layer "F.Cu") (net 11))
 (segment (start 150.274999 113.925001) (end 148.4 115.8) (width 0.3) (layer "F.Cu") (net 11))
 (segment (start 144.6 115.5) (end 144.6 114.2) (width 0.3) (layer "F.Cu") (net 11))
 (segment (start 150.274999 110.125001) (end 150.274999 112.2638) (width 0.3) (layer "F.Cu") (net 11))
 (segment (start 148.4 115.8) (end 148.4 117.1) (width 0.3) (layer "F.Cu") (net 11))
 (segment (start 151.544999 107.3362) (end 151.544999 108.855001) (width 0.3) (layer "F.Cu") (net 11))
 (segment (start 152.814999 107.3362) (end 156.58255 107.3362) (width 0.3) (layer "F.Cu") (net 15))
 (segment (start 156.58255 107.3362) (end 156.7 107.21875) (width 0.3) (layer "F.Cu") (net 15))
 (segment (start 156.7 107.74375) (end 156.7 106.881249) (width 0.3) (layer "F.Cu") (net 15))
 (segment (start 150.274999 103.274999) (end 150 103) (width 0.3) (layer "F.Cu") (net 14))
 (segment (start 150.274999 107.3362) (end 150.274999 103.274999) (width 0.3) (layer "F.Cu") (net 14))
 (segment (start 117.5 123.757763) (end 117.5 137.86) (width 0.5) (layer "F.Cu") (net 2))
 (segment (start 146.8 106.4) (end 146.9 106.3) (width 0.3) (layer "F.Cu") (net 2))
 (segment (start 112.8 121.8) (end 113.678987 121.8) (width 0.3) (layer "F.Cu") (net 2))
 (segment (start 149.004999 106.704999) (end 149.004999 107.3362) (width 0.3) (layer "F.Cu") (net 2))
 (segment (start 147.25 126.15) (end 147.25 129.05) (width 0.3) (layer "F.Cu") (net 2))
 (segment (start 131.9 123.5) (end 117.54 137.86) (width 0.3) (layer "F.Cu") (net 2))
 (segment (start 146.9 103) (end 146.9 106.3) (width 0.3) (layer "F.Cu") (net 2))
 (segment (start 146.9 106.3) (end 149 106.3) (width 0.3) (layer "F.Cu") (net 2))
 (segment (start 152.814999 114.214999) (end 152.814999 112.2638) (width 0.3) (layer "F.Cu") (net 2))
 (segment (start 144.6 123.5) (end 131.9 123.5) (width 0.3) (layer "F.Cu") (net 2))
 (segment (start 117.5 137.86) (end 117.54 137.9) (width 0.3) (layer "F.Cu") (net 2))
 (segment (start 149.004999 106.304999) (end 149.004999 107.3362) (width 0.3) (layer "F.Cu") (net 2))
 (segment (start 117.54 123.797763) (end 117.5 123.757763) (width 0.3) (layer "F.Cu") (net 2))
 (segment (start 149 106.3) (end 149.004999 106.304999) (width 0.3) (layer "F.Cu") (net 2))
 (segment (start 144.6 123.5) (end 147.25 126.15) (width 0.3) (layer "F.Cu") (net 2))
 (segment (start 143.9625 106.4) (end 146.8 106.4) (width 0.3) (layer "F.Cu") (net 2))
 (via (at 144.6 123.5) (size 0.8) (drill 0.4) (layers "F.Cu" "B.Cu") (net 2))
 (via (at 152.814999 114.214999) (size 0.8) (drill 0.4) (layers "F.Cu" "B.Cu") (free yes) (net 2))
 (via (at 146.9 106.3) (size 0.8) (drill 0.4) (layers "F.Cu" "B.Cu") (free yes) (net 2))
 (segment (start 152.814999 114.214999) (end 152.729998 114.3) (width 0.3) (layer "B.Cu") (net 2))
 (segment (start 146.9 114.3) (end 146.9 110.7) (width 0.3) (layer "B.Cu") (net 2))
 (segment (start 144.6 116.6) (end 146.9 114.3) (width 0.3) (layer "B.Cu") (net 2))
 (segment (start 144.6 123.5) (end 144.6 116.6) (width 0.3) (layer "B.Cu") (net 2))
 (segment (start 152.729998 114.3) (end 146.9 114.3) (width 0.3) (layer "B.Cu") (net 2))
 (segment (start 146.9 110.7) (end 146.9 106.3) (width 0.3) (layer "B.Cu") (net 2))
 (segment (start 122.62 137.9) (end 122.62 137.28) (width 0.3) (layer "F.Cu") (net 4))
 (segment (start 145.75 127.85) (end 145.75 129.05) (width 0.3) (layer "F.Cu") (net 4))
 (segment (start 122.62 137.28) (end 133.7 126.2) (width 0.3) (layer "F.Cu") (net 4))
 (segment (start 133.7 126.2) (end 144.1 126.2) (width 0.3) (layer "F.Cu") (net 4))
 (segment (start 144.1 126.2) (end 145.75 127.85) (width 0.3) (layer "F.Cu") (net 4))
 (segment (start 146.25 127.15) (end 146.25 129.05) (width 0.3) (layer "F.Cu") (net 3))
 (segment (start 120.079999 137.520001) (end 132.5 125.1) (width 0.3) (layer "F.Cu") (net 3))
 (segment (start 120.079999 137.9) (end 120.079999 137.520001) (width 0.3) (layer "F.Cu") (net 3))
 (segment (start 144.2 125.1) (end 146.25 127.15) (width 0.3) (layer "F.Cu") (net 3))
 (segment (start 132.5 125.1) (end 144.2 125.1) (width 0.3) (layer "F.Cu") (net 3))
 (segment (start 144.2 127.2) (end 145.25 128.25) (width 0.3) (layer "F.Cu") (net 5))
 (segment (start 135.3 127.2) (end 144.2 127.2) (width 0.3) (layer "F.Cu") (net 5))
 (segment (start 145.25 128.25) (end 145.25 129.05) (width 0.3) (layer "F.Cu") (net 5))
 (segment (start 125.16 137.34) (end 135.3 127.2) (width 0.3) (layer "F.Cu") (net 5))
 (segment (start 125.16 137.9) (end 125.16 137.34) (width 0.3) (layer "F.Cu") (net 5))
 (segment (start 148.25 124.25) (end 142.050264 118.050264) (width 0.3) (layer "F.Cu") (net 8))
 (segment (start 148.25 129.05) (end 148.75 129.05) (width 0.3) (layer "F.Cu") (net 8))
 (segment (start 142.050264 118.050264) (end 133.649736 118.050264) (width 0.3) (layer "F.Cu") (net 8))
 (segment (start 148.25 129.05) (end 148.25 124.25) (width 0.3) (layer "F.Cu") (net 8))
 (segment (start 147.75 129.05) (end 148.25 129.05) (width 0.3) (layer "F.Cu") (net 8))
 (segment (start 133.6 118.1) (end 133.6 115.55) (width 0.3) (layer "F.Cu") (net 8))
 (segment (start 120.55 123.707764) (end 120.6 123.757763) (width 0.25) (layer "F.Cu") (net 9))
 (segment (start 120.55 119.857763) (end 120.55 123.707764) (width 0.25) (layer "F.Cu") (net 9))
 (segment (start 120.749999 119.657764) (end 120.55 119.857763) (width 0.25) (layer "F.Cu") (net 9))
 (segment (start 121.275 119.657764) (end 120.749999 119.657764) (width 0.25) (layer "F.Cu") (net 9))
 (segment (start 151.5 122.5) (end 151.5 117.1) (width 0.3) (layer "F.Cu") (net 12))
 (segment (start 151.544999 117.055001) (end 151.5 117.1) (width 0.3) (layer "F.Cu") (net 12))
 (segment (start 151.544999 112.2638) (end 151.544999 117.055001) (width 0.3) (layer "F.Cu") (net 12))
 (segment (start 146.75 129.95) (end 147.4 130.6) (width 0.3) (layer "F.Cu") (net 7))
 (segment (start 146.75 129.05) (end 146.75 129.95) (width 0.3) (layer "F.Cu") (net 7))
 (segment (start 151.5 123.799998) (end 156.099998 123.799998) (width 0.3) (layer "F.Cu") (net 7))
 (segment (start 156.1 123.8) (end 157.9 123.8) (width 0.3) (layer "F.Cu") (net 7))
 (segment (start 151.5 129.3) (end 151.5 123.799998) (width 0.3) (layer "F.Cu") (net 7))
 (segment (start 150.2 130.6) (end 151.5 129.3) (width 0.3) (layer "F.Cu") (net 7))
 (segment (start 147.4 130.6) (end 150.2 130.6) (width 0.3) (layer "F.Cu") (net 7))
 (segment (start 156.099998 123.799998) (end 156.1 123.8) (width 0.3) (layer "F.Cu") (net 7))
 (segment (start 127.7 118.050264) (end 132.250264 118.050264) (width 0.25) (layer "F.Cu") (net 6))
 (segment (start 117 115.3) (end 120 115.3) (width 0.5) (layer "F.Cu") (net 13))
 (segment (start 120 115.3) (end 120.15 115.15) (width 0.25) (layer "F.Cu") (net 13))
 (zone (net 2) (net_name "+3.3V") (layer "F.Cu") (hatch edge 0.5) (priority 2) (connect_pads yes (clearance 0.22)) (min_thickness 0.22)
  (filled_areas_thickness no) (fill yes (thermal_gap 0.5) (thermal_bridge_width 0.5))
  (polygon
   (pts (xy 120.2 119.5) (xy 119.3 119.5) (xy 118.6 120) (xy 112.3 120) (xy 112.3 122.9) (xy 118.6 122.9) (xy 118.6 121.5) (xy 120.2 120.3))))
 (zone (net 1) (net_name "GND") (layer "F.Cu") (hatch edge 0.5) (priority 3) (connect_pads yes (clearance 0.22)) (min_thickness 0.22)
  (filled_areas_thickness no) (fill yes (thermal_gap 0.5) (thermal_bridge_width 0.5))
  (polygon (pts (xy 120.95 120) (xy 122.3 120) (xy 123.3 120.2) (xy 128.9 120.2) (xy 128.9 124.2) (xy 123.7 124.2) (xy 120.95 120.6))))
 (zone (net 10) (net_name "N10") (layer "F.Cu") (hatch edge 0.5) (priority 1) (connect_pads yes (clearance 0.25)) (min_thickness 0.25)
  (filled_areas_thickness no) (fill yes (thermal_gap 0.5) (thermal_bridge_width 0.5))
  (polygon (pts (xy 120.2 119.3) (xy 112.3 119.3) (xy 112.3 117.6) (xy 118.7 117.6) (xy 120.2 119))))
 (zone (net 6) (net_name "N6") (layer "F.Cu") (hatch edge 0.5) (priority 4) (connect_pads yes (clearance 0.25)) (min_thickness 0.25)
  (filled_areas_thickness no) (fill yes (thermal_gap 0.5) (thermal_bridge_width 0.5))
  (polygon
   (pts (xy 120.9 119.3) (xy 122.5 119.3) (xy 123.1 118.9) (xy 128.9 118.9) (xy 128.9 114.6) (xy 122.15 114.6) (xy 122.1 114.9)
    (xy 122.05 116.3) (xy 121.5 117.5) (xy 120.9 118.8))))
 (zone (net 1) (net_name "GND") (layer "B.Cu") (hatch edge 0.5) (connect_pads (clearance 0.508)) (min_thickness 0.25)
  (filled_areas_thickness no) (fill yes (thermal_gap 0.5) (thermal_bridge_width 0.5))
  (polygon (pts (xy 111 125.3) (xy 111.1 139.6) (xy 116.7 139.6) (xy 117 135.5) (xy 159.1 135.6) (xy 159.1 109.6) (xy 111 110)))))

